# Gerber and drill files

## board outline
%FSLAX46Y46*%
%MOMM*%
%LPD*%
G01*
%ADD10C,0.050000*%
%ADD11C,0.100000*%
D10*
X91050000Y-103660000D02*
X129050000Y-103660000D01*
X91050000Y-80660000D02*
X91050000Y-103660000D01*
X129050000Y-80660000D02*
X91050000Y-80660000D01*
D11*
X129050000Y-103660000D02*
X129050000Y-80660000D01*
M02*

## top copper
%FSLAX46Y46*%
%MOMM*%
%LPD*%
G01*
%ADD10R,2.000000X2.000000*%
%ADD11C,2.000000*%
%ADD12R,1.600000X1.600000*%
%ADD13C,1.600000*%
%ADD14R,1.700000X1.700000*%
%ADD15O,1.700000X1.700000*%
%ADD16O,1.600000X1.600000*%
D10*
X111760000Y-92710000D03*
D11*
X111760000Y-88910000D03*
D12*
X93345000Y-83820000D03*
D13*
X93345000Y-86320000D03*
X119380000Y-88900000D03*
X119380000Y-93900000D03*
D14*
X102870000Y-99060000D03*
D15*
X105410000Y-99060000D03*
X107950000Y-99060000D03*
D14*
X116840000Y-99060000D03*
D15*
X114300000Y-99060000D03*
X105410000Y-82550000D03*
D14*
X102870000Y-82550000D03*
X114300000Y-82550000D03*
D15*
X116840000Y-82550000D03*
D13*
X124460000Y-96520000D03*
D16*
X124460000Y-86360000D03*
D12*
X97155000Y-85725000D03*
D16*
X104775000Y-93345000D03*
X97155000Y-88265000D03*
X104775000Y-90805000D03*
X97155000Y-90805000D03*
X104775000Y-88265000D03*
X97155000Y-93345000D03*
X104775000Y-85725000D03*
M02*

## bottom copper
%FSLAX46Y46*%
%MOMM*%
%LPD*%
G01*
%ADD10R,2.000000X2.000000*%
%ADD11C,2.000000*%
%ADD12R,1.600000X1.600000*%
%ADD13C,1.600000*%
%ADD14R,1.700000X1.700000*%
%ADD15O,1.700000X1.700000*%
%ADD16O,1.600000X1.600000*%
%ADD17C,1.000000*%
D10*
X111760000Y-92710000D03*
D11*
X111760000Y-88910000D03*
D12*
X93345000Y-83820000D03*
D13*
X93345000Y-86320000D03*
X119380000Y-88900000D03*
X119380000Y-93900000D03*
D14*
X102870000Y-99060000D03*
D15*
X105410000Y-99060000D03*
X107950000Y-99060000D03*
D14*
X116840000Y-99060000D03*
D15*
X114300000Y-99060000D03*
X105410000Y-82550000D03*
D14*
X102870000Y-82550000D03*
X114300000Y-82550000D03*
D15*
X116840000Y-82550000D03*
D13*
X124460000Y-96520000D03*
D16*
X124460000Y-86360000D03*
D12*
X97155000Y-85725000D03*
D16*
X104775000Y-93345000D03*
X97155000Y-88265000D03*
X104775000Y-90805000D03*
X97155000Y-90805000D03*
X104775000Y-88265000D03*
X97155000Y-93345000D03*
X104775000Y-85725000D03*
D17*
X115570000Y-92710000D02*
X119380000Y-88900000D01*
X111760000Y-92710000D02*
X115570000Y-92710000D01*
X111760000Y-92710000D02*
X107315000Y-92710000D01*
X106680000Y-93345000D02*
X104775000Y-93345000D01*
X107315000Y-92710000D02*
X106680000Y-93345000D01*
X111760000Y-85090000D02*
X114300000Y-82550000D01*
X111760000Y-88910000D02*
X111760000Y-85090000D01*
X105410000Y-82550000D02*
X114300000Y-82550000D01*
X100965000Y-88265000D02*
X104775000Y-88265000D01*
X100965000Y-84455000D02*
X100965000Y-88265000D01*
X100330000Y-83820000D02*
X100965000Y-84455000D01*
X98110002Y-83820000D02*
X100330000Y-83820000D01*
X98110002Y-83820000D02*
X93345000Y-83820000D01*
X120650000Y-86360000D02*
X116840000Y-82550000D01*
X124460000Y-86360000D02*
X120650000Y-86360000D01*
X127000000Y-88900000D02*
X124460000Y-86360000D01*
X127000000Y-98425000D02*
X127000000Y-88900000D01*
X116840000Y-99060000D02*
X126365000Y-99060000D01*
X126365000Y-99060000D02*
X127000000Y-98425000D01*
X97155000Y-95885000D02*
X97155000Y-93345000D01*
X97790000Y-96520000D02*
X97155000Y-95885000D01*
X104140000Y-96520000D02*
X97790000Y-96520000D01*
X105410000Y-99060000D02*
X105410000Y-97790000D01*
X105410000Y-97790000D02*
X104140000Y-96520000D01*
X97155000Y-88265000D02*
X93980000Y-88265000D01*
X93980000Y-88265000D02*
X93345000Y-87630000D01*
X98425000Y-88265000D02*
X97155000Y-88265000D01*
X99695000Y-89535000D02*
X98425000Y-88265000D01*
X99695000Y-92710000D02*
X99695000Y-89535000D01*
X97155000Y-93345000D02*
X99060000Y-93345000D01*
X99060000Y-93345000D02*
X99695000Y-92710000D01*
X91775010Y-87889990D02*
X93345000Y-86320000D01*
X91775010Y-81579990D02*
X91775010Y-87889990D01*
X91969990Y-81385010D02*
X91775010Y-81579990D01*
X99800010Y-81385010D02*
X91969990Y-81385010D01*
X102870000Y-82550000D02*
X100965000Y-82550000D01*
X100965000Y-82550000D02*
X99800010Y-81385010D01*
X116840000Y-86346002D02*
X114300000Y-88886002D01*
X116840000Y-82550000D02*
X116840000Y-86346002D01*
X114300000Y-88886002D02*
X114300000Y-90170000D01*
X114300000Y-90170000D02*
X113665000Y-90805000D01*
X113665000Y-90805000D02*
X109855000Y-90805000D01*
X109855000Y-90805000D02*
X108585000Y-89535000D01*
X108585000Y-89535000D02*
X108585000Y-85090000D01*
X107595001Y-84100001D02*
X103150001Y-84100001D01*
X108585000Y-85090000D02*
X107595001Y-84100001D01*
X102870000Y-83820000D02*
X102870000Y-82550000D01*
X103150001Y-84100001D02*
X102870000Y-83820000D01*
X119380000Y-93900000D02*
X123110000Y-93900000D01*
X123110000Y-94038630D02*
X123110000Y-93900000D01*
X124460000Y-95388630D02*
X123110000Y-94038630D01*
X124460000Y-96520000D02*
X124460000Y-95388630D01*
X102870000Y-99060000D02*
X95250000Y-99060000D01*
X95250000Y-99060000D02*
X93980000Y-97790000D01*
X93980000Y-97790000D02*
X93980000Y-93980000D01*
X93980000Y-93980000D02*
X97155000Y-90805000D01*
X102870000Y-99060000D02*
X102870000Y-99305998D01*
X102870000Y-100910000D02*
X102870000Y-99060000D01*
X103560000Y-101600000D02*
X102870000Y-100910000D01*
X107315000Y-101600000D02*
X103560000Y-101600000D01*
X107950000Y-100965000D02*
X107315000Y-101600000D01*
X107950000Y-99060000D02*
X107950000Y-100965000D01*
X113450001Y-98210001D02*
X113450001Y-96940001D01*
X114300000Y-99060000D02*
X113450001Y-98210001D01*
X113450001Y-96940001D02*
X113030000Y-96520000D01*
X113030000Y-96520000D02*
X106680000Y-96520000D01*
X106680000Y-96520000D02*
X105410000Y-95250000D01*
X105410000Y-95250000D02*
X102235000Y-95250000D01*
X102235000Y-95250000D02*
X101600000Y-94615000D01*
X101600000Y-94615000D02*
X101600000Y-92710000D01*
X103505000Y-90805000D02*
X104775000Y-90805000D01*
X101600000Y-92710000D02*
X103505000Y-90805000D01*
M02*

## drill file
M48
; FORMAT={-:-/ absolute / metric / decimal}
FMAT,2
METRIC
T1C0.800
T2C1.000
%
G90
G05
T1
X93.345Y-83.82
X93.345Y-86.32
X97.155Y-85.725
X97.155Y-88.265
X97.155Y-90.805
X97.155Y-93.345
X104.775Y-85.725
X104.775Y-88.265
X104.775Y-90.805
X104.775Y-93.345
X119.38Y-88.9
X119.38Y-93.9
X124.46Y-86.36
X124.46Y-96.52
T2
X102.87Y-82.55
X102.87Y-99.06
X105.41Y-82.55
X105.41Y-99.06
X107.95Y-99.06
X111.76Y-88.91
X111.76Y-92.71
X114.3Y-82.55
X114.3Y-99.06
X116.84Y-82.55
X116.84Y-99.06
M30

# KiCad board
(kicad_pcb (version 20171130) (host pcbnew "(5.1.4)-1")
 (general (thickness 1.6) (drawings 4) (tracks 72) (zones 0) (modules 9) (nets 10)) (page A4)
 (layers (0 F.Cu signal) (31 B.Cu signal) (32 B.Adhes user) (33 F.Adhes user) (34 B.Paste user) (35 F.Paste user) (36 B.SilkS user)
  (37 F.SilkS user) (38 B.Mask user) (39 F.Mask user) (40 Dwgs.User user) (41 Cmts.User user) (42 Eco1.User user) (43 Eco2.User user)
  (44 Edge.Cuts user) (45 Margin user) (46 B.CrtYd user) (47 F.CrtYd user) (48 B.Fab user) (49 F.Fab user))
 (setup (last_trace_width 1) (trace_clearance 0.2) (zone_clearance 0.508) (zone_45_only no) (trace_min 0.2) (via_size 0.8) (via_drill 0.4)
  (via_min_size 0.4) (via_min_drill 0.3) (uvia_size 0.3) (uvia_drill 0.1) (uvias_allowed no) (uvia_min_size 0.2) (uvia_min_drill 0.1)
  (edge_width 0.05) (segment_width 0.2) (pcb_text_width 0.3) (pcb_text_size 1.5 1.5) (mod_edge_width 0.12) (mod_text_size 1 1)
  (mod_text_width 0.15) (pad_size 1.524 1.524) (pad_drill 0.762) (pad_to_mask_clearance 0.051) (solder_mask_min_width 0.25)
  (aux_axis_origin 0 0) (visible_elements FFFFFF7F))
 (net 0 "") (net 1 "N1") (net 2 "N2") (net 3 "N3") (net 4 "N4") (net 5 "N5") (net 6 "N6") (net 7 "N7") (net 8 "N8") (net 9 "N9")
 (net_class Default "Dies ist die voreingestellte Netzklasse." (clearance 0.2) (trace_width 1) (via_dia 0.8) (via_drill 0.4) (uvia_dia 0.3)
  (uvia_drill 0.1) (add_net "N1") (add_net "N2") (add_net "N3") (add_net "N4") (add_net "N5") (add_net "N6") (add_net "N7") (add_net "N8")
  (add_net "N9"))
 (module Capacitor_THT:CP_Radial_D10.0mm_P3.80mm (layer F.Cu) (at 111.76 92.71 90)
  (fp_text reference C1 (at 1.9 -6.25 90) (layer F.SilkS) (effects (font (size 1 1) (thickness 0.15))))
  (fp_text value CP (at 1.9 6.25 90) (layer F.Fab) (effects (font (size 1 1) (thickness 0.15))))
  (pad 1 thru_hole rect (at 0 0 90) (size 2 2) (drill 1) (layers *.Cu *.Mask) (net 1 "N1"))
  (pad 2 thru_hole circle (at 3.8 0 90) (size 2 2) (drill 1) (layers *.Cu *.Mask) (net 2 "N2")))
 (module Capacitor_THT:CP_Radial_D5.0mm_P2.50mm (layer F.Cu) (at 93.345 83.82 270)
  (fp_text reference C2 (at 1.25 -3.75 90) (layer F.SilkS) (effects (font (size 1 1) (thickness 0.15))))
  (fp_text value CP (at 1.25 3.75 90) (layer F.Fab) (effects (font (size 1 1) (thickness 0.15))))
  (pad 1 thru_hole rect (at 0 0 270) (size 1.6 1.6) (drill 0.8) (layers *.Cu *.Mask) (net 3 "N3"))
  (pad 2 thru_hole circle (at 2.5 0 270) (size 1.6 1.6) (drill 0.8) (layers *.Cu *.Mask) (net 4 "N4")))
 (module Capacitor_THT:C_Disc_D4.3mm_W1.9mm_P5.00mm (layer F.Cu) (at 119.38 88.9 270)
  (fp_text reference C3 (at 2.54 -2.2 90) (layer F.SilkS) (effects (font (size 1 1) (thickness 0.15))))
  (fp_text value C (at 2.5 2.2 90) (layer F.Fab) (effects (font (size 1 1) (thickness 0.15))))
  (pad 1 thru_hole circle (at 0 0 270) (size 1.6 1.6) (drill 0.8) (layers *.Cu *.Mask) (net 1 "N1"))
  (pad 2 thru_hole circle (at 5 0 270) (size 1.6 1.6) (drill 0.8) (layers *.Cu *.Mask) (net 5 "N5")))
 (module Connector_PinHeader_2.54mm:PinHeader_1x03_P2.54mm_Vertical (layer F.Cu) (at 102.87 99.06 90)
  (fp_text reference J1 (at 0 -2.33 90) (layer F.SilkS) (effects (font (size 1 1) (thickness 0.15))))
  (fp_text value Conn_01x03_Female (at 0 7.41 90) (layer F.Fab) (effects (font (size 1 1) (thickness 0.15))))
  (pad 1 thru_hole rect (at 0 0 90) (size 1.7 1.7) (drill 1) (layers *.Cu *.Mask) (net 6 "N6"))
  (pad 2 thru_hole oval (at 0 2.54 90) (size 1.7 1.7) (drill 1) (layers *.Cu *.Mask) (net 4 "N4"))
  (pad 3 thru_hole oval (at 0 5.08 90) (size 1.7 1.7) (drill 1) (layers *.Cu *.Mask) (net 6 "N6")))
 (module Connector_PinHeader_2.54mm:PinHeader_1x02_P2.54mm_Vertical (layer F.Cu) (at 116.84 99.06 270)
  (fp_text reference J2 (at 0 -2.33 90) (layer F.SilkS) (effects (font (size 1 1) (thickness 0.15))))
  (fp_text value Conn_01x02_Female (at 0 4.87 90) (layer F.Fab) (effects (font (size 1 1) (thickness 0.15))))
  (pad 1 thru_hole rect (at 0 0 270) (size 1.7 1.7) (drill 1) (layers *.Cu *.Mask) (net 4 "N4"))
  (pad 2 thru_hole oval (at 0 2.54 270) (size 1.7 1.7) (drill 1) (layers *.Cu *.Mask) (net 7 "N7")))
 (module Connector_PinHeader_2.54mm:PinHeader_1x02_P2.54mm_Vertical (layer F.Cu) (at 102.87 82.55 90)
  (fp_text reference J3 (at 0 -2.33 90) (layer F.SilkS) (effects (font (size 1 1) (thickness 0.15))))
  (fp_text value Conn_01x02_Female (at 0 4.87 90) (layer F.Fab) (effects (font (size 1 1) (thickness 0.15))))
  (pad 2 thru_hole oval (at 0 2.54 90) (size 1.7 1.7) (drill 1) (layers *.Cu *.Mask) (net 2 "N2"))
  (pad 1 thru_hole rect (at 0 0 90) (size 1.7 1.7) (drill 1) (layers *.Cu *.Mask) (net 4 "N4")))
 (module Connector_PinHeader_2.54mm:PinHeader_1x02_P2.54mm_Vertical (layer F.Cu) (at 114.3 82.55 90)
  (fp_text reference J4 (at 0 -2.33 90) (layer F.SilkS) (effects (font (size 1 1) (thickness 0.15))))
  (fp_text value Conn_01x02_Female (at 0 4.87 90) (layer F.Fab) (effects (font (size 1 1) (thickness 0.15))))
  (pad 1 thru_hole rect (at 0 0 90) (size 1.7 1.7) (drill 1) (layers *.Cu *.Mask) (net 2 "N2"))
  (pad 2 thru_hole oval (at 0 2.54 90) (size 1.7 1.7) (drill 1) (layers *.Cu *.Mask) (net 4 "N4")))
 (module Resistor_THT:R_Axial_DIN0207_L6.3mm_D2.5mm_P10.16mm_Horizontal (layer F.Cu) (at 124.46 96.52 90)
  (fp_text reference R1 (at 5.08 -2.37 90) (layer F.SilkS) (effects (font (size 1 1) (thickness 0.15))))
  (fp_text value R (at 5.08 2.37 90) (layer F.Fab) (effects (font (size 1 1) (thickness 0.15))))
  (pad 1 thru_hole circle (at 0 0 90) (size 1.6 1.6) (drill 0.8) (layers *.Cu *.Mask) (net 5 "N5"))
  (pad 2 thru_hole oval (at 10.16 0 90) (size 1.6 1.6) (drill 0.8) (layers *.Cu *.Mask) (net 4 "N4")))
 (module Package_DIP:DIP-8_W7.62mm (layer F.Cu) (at 97.155 85.725)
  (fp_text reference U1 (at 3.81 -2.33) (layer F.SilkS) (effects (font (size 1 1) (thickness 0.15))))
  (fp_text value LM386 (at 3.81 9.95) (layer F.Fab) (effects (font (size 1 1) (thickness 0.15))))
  (pad 1 thru_hole rect (at 0 0) (size 1.6 1.6) (drill 0.8) (layers *.Cu *.Mask) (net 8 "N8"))
  (pad 5 thru_hole oval (at 7.62 7.62) (size 1.6 1.6) (drill 0.8) (layers *.Cu *.Mask) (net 1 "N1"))
  (pad 2 thru_hole oval (at 0 2.54) (size 1.6 1.6) (drill 0.8) (layers *.Cu *.Mask) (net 4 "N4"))
  (pad 6 thru_hole oval (at 7.62 5.08) (size 1.6 1.6) (drill 0.8) (layers *.Cu *.Mask) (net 7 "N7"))
  (pad 3 thru_hole oval (at 0 5.08) (size 1.6 1.6) (drill 0.8) (layers *.Cu *.Mask) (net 6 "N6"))
  (pad 7 thru_hole oval (at 7.62 2.54) (size 1.6 1.6) (drill 0.8) (layers *.Cu *.Mask) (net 3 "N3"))
  (pad 4 thru_hole oval (at 0 7.62) (size 1.6 1.6) (drill 0.8) (layers *.Cu *.Mask) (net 4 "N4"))
  (pad 8 thru_hole oval (at 7.62 0) (size 1.6 1.6) (drill 0.8) (layers *.Cu *.Mask) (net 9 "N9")))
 (gr_line (start 91.05 103.66) (end 129.05 103.66) (layer Edge.Cuts) (width 0.05))
 (gr_line (start 91.05 80.66) (end 91.05 103.66) (layer Edge.Cuts) (width 0.05))
 (gr_line (start 129.05 80.66) (end 91.05 80.66) (layer Edge.Cuts) (width 0.05))
 (gr_line (start 129.05 103.66) (end 129.05 80.66) (layer Edge.Cuts) (width 0.1))
 (segment (start 115.57 92.71) (end 119.38 88.9) (width 1) (layer B.Cu) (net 1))
 (segment (start 111.76 92.71) (end 115.57 92.71) (width 1) (layer B.Cu) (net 1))
 (segment (start 111.76 92.71) (end 107.315 92.71) (width 1) (layer B.Cu) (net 1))
 (segment (start 106.68 93.345) (end 104.775 93.345) (width 1) (layer B.Cu) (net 1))
 (segment (start 107.315 92.71) (end 106.68 93.345) (width 1) (layer B.Cu) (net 1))
 (segment (start 111.76 85.09) (end 114.3 82.55) (width 1) (layer B.Cu) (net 2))
 (segment (start 111.76 88.91) (end 111.76 85.09) (width 1) (layer B.Cu) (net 2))
 (segment (start 105.41 82.55) (end 114.3 82.55) (width 1) (layer B.Cu) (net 2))
 (segment (start 100.965 88.265) (end 104.775 88.265) (width 1) (layer B.Cu) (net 3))
 (segment (start 100.965 84.455) (end 100.965 88.265) (width 1) (layer B.Cu) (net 3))
 (segment (start 100.33 83.82) (end 100.965 84.455) (width 1) (layer B.Cu) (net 3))
 (segment (start 98.110002 83.82) (end 100.33 83.82) (width 1) (layer B.Cu) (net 3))
 (segment (start 98.110002 83.82) (end 93.345 83.82) (width 1) (layer B.Cu) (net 3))
 (segment (start 120.65 86.36) (end 116.84 82.55) (width 1) (layer B.Cu) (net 4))
 (segment (start 124.46 86.36) (end 120.65 86.36) (width 1) (layer B.Cu) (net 4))
 (segment (start 127 88.9) (end 124.46 86.36) (width 1) (layer B.Cu) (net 4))
 (segment (start 127 98.425) (end 127 88.9) (width 1) (layer B.Cu) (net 4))
 (segment (start 116.84 99.06) (end 126.365 99.06) (width 1) (layer B.Cu) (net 4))
 (segment (start 126.365 99.06) (end 127 98.425) (width 1) (layer B.Cu) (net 4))
 (segment (start 97.155 95.885) (end 97.155 93.345) (width 1) (layer B.Cu) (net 4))
 (segment (start 97.79 96.52) (end 97.155 95.885) (width 1) (layer B.Cu) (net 4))
 (segment (start 104.14 96.52) (end 97.79 96.52) (width 1) (layer B.Cu) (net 4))
 (segment (start 105.41 99.06) (end 105.41 97.79) (width 1) (layer B.Cu) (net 4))
 (segment (start 105.41 97.79) (end 104.14 96.52) (width 1) (layer B.Cu) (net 4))
 (segment (start 97.155 88.265) (end 93.98 88.265) (width 1) (layer B.Cu) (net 4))
 (segment (start 93.98 88.265) (end 93.345 87.63) (width 1) (layer B.Cu) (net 4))
 (segment (start 98.425 88.265) (end 97.155 88.265) (width 1) (layer B.Cu) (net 4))
 (segment (start 99.695 89.535) (end 98.425 88.265) (width 1) (layer B.Cu) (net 4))
 (segment (start 99.695 92.71) (end 99.695 89.535) (width 1) (layer B.Cu) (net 4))
 (segment (start 97.155 93.345) (end 99.06 93.345) (width 1) (layer B.Cu) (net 4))
 (segment (start 99.06 93.345) (end 99.695 92.71) (width 1) (layer B.Cu) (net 4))
 (segment (start 91.77501 87.88999) (end 93.345 86.32) (width 1) (layer B.Cu) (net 4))
 (segment (start 91.77501 81.57999) (end 91.77501 87.88999) (width 1) (layer B.Cu) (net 4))
 (segment (start 91.96999 81.38501) (end 91.77501 81.57999) (width 1) (layer B.Cu) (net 4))
 (segment (start 99.80001 81.38501) (end 91.96999 81.38501) (width 1) (layer B.Cu) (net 4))
 (segment (start 102.87 82.55) (end 100.965 82.55) (width 1) (layer B.Cu) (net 4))
 (segment (start 100.965 82.55) (end 99.80001 81.38501) (width 1) (layer B.Cu) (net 4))
 (segment (start 116.84 86.346002) (end 114.3 88.886002) (width 1) (layer B.Cu) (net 4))
 (segment (start 116.84 82.55) (end 116.84 86.346002) (width 1) (layer B.Cu) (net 4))
 (segment (start 114.3 88.886002) (end 114.3 90.17) (width 1) (layer B.Cu) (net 4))
 (segment (start 114.3 90.17) (end 113.665 90.805) (width 1) (layer B.Cu) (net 4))
 (segment (start 113.665 90.805) (end 109.855 90.805) (width 1) (layer B.Cu) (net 4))
 (segment (start 109.855 90.805) (end 108.585 89.535) (width 1) (layer B.Cu) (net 4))
 (segment (start 108.585 89.535) (end 108.585 85.09) (width 1) (layer B.Cu) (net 4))
 (segment (start 107.595001 84.100001) (end 103.150001 84.100001) (width 1) (layer B.Cu) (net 4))
 (segment (start 108.585 85.09) (end 107.595001 84.100001) (width 1) (layer B.Cu) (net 4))
 (segment (start 102.87 83.82) (end 102.87 82.55) (width 1) (layer B.Cu) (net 4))
 (segment (start 103.150001 84.100001) (end 102.87 83.82) (width 1) (layer B.Cu) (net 4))
 (segment (start 119.38 93.9) (end 123.11 93.9) (width 1) (layer B.Cu) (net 5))
 (segment (start 123.11 94.03863) (end 123.11 93.9) (width 1) (layer B.Cu) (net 5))
 (segment (start 124.46 95.38863) (end 123.11 94.03863) (width 1) (layer B.Cu) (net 5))
 (segment (start 124.46 96.52) (end 124.46 95.38863) (width 1) (layer B.Cu) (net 5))
 (segment (start 102.87 99.06) (end 95.25 99.06) (width 1) (layer B.Cu) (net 6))
 (segment (start 95.25 99.06) (end 93.98 97.79) (width 1) (layer B.Cu) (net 6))
 (segment (start 93.98 97.79) (end 93.98 93.98) (width 1) (layer B.Cu) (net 6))
 (segment (start 93.98 93.98) (end 97.155 90.805) (width 1) (layer B.Cu) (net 6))
 (segment (start 102.87 99.06) (end 102.87 99.305998) (width 1) (layer B.Cu) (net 6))
 (segment (start 102.87 100.91) (end 102.87 99.06) (width 1) (layer B.Cu) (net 6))
 (segment (start 103.56 101.6) (end 102.87 100.91) (width 1) (layer B.Cu) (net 6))
 (segment (start 107.315 101.6) (end 103.56 101.6) (width 1) (layer B.Cu) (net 6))
 (segment (start 107.95 100.965) (end 107.315 101.6) (width 1) (layer B.Cu) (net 6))
 (segment (start 107.95 99.06) (end 107.95 100.965) (width 1) (layer B.Cu) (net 6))
 (segment (start 113.450001 98.210001) (end 113.450001 96.940001) (width 1) (layer B.Cu) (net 7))
 (segment (start 114.3 99.06) (end 113.450001 98.210001) (width 1) (layer B.Cu) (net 7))
 (segment (start 113.450001 96.940001) (end 113.03 96.52) (width 1) (layer B.Cu) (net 7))
 (segment (start 113.03 96.52) (end 106.68 96.52) (width 1) (layer B.Cu) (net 7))
 (segment (start 106.68 96.52) (end 105.41 95.25) (width 1) (layer B.Cu) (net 7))
 (segment (start 105.41 95.25) (end 102.235 95.25) (width 1) (layer B.Cu) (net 7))
 (segment (start 102.235 95.25) (end 101.6 94.615) (width 1) (layer B.Cu) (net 7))
 (segment (start 101.6 94.615) (end 101.6 92.71) (width 1) (layer B.Cu) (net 7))
 (segment (start 103.505 90.805) (end 104.775 90.805) (width 1) (layer B.Cu) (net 7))
 (segment (start 101.6 92.71) (end 103.505 90.805) (width 1) (layer B.Cu) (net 7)))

